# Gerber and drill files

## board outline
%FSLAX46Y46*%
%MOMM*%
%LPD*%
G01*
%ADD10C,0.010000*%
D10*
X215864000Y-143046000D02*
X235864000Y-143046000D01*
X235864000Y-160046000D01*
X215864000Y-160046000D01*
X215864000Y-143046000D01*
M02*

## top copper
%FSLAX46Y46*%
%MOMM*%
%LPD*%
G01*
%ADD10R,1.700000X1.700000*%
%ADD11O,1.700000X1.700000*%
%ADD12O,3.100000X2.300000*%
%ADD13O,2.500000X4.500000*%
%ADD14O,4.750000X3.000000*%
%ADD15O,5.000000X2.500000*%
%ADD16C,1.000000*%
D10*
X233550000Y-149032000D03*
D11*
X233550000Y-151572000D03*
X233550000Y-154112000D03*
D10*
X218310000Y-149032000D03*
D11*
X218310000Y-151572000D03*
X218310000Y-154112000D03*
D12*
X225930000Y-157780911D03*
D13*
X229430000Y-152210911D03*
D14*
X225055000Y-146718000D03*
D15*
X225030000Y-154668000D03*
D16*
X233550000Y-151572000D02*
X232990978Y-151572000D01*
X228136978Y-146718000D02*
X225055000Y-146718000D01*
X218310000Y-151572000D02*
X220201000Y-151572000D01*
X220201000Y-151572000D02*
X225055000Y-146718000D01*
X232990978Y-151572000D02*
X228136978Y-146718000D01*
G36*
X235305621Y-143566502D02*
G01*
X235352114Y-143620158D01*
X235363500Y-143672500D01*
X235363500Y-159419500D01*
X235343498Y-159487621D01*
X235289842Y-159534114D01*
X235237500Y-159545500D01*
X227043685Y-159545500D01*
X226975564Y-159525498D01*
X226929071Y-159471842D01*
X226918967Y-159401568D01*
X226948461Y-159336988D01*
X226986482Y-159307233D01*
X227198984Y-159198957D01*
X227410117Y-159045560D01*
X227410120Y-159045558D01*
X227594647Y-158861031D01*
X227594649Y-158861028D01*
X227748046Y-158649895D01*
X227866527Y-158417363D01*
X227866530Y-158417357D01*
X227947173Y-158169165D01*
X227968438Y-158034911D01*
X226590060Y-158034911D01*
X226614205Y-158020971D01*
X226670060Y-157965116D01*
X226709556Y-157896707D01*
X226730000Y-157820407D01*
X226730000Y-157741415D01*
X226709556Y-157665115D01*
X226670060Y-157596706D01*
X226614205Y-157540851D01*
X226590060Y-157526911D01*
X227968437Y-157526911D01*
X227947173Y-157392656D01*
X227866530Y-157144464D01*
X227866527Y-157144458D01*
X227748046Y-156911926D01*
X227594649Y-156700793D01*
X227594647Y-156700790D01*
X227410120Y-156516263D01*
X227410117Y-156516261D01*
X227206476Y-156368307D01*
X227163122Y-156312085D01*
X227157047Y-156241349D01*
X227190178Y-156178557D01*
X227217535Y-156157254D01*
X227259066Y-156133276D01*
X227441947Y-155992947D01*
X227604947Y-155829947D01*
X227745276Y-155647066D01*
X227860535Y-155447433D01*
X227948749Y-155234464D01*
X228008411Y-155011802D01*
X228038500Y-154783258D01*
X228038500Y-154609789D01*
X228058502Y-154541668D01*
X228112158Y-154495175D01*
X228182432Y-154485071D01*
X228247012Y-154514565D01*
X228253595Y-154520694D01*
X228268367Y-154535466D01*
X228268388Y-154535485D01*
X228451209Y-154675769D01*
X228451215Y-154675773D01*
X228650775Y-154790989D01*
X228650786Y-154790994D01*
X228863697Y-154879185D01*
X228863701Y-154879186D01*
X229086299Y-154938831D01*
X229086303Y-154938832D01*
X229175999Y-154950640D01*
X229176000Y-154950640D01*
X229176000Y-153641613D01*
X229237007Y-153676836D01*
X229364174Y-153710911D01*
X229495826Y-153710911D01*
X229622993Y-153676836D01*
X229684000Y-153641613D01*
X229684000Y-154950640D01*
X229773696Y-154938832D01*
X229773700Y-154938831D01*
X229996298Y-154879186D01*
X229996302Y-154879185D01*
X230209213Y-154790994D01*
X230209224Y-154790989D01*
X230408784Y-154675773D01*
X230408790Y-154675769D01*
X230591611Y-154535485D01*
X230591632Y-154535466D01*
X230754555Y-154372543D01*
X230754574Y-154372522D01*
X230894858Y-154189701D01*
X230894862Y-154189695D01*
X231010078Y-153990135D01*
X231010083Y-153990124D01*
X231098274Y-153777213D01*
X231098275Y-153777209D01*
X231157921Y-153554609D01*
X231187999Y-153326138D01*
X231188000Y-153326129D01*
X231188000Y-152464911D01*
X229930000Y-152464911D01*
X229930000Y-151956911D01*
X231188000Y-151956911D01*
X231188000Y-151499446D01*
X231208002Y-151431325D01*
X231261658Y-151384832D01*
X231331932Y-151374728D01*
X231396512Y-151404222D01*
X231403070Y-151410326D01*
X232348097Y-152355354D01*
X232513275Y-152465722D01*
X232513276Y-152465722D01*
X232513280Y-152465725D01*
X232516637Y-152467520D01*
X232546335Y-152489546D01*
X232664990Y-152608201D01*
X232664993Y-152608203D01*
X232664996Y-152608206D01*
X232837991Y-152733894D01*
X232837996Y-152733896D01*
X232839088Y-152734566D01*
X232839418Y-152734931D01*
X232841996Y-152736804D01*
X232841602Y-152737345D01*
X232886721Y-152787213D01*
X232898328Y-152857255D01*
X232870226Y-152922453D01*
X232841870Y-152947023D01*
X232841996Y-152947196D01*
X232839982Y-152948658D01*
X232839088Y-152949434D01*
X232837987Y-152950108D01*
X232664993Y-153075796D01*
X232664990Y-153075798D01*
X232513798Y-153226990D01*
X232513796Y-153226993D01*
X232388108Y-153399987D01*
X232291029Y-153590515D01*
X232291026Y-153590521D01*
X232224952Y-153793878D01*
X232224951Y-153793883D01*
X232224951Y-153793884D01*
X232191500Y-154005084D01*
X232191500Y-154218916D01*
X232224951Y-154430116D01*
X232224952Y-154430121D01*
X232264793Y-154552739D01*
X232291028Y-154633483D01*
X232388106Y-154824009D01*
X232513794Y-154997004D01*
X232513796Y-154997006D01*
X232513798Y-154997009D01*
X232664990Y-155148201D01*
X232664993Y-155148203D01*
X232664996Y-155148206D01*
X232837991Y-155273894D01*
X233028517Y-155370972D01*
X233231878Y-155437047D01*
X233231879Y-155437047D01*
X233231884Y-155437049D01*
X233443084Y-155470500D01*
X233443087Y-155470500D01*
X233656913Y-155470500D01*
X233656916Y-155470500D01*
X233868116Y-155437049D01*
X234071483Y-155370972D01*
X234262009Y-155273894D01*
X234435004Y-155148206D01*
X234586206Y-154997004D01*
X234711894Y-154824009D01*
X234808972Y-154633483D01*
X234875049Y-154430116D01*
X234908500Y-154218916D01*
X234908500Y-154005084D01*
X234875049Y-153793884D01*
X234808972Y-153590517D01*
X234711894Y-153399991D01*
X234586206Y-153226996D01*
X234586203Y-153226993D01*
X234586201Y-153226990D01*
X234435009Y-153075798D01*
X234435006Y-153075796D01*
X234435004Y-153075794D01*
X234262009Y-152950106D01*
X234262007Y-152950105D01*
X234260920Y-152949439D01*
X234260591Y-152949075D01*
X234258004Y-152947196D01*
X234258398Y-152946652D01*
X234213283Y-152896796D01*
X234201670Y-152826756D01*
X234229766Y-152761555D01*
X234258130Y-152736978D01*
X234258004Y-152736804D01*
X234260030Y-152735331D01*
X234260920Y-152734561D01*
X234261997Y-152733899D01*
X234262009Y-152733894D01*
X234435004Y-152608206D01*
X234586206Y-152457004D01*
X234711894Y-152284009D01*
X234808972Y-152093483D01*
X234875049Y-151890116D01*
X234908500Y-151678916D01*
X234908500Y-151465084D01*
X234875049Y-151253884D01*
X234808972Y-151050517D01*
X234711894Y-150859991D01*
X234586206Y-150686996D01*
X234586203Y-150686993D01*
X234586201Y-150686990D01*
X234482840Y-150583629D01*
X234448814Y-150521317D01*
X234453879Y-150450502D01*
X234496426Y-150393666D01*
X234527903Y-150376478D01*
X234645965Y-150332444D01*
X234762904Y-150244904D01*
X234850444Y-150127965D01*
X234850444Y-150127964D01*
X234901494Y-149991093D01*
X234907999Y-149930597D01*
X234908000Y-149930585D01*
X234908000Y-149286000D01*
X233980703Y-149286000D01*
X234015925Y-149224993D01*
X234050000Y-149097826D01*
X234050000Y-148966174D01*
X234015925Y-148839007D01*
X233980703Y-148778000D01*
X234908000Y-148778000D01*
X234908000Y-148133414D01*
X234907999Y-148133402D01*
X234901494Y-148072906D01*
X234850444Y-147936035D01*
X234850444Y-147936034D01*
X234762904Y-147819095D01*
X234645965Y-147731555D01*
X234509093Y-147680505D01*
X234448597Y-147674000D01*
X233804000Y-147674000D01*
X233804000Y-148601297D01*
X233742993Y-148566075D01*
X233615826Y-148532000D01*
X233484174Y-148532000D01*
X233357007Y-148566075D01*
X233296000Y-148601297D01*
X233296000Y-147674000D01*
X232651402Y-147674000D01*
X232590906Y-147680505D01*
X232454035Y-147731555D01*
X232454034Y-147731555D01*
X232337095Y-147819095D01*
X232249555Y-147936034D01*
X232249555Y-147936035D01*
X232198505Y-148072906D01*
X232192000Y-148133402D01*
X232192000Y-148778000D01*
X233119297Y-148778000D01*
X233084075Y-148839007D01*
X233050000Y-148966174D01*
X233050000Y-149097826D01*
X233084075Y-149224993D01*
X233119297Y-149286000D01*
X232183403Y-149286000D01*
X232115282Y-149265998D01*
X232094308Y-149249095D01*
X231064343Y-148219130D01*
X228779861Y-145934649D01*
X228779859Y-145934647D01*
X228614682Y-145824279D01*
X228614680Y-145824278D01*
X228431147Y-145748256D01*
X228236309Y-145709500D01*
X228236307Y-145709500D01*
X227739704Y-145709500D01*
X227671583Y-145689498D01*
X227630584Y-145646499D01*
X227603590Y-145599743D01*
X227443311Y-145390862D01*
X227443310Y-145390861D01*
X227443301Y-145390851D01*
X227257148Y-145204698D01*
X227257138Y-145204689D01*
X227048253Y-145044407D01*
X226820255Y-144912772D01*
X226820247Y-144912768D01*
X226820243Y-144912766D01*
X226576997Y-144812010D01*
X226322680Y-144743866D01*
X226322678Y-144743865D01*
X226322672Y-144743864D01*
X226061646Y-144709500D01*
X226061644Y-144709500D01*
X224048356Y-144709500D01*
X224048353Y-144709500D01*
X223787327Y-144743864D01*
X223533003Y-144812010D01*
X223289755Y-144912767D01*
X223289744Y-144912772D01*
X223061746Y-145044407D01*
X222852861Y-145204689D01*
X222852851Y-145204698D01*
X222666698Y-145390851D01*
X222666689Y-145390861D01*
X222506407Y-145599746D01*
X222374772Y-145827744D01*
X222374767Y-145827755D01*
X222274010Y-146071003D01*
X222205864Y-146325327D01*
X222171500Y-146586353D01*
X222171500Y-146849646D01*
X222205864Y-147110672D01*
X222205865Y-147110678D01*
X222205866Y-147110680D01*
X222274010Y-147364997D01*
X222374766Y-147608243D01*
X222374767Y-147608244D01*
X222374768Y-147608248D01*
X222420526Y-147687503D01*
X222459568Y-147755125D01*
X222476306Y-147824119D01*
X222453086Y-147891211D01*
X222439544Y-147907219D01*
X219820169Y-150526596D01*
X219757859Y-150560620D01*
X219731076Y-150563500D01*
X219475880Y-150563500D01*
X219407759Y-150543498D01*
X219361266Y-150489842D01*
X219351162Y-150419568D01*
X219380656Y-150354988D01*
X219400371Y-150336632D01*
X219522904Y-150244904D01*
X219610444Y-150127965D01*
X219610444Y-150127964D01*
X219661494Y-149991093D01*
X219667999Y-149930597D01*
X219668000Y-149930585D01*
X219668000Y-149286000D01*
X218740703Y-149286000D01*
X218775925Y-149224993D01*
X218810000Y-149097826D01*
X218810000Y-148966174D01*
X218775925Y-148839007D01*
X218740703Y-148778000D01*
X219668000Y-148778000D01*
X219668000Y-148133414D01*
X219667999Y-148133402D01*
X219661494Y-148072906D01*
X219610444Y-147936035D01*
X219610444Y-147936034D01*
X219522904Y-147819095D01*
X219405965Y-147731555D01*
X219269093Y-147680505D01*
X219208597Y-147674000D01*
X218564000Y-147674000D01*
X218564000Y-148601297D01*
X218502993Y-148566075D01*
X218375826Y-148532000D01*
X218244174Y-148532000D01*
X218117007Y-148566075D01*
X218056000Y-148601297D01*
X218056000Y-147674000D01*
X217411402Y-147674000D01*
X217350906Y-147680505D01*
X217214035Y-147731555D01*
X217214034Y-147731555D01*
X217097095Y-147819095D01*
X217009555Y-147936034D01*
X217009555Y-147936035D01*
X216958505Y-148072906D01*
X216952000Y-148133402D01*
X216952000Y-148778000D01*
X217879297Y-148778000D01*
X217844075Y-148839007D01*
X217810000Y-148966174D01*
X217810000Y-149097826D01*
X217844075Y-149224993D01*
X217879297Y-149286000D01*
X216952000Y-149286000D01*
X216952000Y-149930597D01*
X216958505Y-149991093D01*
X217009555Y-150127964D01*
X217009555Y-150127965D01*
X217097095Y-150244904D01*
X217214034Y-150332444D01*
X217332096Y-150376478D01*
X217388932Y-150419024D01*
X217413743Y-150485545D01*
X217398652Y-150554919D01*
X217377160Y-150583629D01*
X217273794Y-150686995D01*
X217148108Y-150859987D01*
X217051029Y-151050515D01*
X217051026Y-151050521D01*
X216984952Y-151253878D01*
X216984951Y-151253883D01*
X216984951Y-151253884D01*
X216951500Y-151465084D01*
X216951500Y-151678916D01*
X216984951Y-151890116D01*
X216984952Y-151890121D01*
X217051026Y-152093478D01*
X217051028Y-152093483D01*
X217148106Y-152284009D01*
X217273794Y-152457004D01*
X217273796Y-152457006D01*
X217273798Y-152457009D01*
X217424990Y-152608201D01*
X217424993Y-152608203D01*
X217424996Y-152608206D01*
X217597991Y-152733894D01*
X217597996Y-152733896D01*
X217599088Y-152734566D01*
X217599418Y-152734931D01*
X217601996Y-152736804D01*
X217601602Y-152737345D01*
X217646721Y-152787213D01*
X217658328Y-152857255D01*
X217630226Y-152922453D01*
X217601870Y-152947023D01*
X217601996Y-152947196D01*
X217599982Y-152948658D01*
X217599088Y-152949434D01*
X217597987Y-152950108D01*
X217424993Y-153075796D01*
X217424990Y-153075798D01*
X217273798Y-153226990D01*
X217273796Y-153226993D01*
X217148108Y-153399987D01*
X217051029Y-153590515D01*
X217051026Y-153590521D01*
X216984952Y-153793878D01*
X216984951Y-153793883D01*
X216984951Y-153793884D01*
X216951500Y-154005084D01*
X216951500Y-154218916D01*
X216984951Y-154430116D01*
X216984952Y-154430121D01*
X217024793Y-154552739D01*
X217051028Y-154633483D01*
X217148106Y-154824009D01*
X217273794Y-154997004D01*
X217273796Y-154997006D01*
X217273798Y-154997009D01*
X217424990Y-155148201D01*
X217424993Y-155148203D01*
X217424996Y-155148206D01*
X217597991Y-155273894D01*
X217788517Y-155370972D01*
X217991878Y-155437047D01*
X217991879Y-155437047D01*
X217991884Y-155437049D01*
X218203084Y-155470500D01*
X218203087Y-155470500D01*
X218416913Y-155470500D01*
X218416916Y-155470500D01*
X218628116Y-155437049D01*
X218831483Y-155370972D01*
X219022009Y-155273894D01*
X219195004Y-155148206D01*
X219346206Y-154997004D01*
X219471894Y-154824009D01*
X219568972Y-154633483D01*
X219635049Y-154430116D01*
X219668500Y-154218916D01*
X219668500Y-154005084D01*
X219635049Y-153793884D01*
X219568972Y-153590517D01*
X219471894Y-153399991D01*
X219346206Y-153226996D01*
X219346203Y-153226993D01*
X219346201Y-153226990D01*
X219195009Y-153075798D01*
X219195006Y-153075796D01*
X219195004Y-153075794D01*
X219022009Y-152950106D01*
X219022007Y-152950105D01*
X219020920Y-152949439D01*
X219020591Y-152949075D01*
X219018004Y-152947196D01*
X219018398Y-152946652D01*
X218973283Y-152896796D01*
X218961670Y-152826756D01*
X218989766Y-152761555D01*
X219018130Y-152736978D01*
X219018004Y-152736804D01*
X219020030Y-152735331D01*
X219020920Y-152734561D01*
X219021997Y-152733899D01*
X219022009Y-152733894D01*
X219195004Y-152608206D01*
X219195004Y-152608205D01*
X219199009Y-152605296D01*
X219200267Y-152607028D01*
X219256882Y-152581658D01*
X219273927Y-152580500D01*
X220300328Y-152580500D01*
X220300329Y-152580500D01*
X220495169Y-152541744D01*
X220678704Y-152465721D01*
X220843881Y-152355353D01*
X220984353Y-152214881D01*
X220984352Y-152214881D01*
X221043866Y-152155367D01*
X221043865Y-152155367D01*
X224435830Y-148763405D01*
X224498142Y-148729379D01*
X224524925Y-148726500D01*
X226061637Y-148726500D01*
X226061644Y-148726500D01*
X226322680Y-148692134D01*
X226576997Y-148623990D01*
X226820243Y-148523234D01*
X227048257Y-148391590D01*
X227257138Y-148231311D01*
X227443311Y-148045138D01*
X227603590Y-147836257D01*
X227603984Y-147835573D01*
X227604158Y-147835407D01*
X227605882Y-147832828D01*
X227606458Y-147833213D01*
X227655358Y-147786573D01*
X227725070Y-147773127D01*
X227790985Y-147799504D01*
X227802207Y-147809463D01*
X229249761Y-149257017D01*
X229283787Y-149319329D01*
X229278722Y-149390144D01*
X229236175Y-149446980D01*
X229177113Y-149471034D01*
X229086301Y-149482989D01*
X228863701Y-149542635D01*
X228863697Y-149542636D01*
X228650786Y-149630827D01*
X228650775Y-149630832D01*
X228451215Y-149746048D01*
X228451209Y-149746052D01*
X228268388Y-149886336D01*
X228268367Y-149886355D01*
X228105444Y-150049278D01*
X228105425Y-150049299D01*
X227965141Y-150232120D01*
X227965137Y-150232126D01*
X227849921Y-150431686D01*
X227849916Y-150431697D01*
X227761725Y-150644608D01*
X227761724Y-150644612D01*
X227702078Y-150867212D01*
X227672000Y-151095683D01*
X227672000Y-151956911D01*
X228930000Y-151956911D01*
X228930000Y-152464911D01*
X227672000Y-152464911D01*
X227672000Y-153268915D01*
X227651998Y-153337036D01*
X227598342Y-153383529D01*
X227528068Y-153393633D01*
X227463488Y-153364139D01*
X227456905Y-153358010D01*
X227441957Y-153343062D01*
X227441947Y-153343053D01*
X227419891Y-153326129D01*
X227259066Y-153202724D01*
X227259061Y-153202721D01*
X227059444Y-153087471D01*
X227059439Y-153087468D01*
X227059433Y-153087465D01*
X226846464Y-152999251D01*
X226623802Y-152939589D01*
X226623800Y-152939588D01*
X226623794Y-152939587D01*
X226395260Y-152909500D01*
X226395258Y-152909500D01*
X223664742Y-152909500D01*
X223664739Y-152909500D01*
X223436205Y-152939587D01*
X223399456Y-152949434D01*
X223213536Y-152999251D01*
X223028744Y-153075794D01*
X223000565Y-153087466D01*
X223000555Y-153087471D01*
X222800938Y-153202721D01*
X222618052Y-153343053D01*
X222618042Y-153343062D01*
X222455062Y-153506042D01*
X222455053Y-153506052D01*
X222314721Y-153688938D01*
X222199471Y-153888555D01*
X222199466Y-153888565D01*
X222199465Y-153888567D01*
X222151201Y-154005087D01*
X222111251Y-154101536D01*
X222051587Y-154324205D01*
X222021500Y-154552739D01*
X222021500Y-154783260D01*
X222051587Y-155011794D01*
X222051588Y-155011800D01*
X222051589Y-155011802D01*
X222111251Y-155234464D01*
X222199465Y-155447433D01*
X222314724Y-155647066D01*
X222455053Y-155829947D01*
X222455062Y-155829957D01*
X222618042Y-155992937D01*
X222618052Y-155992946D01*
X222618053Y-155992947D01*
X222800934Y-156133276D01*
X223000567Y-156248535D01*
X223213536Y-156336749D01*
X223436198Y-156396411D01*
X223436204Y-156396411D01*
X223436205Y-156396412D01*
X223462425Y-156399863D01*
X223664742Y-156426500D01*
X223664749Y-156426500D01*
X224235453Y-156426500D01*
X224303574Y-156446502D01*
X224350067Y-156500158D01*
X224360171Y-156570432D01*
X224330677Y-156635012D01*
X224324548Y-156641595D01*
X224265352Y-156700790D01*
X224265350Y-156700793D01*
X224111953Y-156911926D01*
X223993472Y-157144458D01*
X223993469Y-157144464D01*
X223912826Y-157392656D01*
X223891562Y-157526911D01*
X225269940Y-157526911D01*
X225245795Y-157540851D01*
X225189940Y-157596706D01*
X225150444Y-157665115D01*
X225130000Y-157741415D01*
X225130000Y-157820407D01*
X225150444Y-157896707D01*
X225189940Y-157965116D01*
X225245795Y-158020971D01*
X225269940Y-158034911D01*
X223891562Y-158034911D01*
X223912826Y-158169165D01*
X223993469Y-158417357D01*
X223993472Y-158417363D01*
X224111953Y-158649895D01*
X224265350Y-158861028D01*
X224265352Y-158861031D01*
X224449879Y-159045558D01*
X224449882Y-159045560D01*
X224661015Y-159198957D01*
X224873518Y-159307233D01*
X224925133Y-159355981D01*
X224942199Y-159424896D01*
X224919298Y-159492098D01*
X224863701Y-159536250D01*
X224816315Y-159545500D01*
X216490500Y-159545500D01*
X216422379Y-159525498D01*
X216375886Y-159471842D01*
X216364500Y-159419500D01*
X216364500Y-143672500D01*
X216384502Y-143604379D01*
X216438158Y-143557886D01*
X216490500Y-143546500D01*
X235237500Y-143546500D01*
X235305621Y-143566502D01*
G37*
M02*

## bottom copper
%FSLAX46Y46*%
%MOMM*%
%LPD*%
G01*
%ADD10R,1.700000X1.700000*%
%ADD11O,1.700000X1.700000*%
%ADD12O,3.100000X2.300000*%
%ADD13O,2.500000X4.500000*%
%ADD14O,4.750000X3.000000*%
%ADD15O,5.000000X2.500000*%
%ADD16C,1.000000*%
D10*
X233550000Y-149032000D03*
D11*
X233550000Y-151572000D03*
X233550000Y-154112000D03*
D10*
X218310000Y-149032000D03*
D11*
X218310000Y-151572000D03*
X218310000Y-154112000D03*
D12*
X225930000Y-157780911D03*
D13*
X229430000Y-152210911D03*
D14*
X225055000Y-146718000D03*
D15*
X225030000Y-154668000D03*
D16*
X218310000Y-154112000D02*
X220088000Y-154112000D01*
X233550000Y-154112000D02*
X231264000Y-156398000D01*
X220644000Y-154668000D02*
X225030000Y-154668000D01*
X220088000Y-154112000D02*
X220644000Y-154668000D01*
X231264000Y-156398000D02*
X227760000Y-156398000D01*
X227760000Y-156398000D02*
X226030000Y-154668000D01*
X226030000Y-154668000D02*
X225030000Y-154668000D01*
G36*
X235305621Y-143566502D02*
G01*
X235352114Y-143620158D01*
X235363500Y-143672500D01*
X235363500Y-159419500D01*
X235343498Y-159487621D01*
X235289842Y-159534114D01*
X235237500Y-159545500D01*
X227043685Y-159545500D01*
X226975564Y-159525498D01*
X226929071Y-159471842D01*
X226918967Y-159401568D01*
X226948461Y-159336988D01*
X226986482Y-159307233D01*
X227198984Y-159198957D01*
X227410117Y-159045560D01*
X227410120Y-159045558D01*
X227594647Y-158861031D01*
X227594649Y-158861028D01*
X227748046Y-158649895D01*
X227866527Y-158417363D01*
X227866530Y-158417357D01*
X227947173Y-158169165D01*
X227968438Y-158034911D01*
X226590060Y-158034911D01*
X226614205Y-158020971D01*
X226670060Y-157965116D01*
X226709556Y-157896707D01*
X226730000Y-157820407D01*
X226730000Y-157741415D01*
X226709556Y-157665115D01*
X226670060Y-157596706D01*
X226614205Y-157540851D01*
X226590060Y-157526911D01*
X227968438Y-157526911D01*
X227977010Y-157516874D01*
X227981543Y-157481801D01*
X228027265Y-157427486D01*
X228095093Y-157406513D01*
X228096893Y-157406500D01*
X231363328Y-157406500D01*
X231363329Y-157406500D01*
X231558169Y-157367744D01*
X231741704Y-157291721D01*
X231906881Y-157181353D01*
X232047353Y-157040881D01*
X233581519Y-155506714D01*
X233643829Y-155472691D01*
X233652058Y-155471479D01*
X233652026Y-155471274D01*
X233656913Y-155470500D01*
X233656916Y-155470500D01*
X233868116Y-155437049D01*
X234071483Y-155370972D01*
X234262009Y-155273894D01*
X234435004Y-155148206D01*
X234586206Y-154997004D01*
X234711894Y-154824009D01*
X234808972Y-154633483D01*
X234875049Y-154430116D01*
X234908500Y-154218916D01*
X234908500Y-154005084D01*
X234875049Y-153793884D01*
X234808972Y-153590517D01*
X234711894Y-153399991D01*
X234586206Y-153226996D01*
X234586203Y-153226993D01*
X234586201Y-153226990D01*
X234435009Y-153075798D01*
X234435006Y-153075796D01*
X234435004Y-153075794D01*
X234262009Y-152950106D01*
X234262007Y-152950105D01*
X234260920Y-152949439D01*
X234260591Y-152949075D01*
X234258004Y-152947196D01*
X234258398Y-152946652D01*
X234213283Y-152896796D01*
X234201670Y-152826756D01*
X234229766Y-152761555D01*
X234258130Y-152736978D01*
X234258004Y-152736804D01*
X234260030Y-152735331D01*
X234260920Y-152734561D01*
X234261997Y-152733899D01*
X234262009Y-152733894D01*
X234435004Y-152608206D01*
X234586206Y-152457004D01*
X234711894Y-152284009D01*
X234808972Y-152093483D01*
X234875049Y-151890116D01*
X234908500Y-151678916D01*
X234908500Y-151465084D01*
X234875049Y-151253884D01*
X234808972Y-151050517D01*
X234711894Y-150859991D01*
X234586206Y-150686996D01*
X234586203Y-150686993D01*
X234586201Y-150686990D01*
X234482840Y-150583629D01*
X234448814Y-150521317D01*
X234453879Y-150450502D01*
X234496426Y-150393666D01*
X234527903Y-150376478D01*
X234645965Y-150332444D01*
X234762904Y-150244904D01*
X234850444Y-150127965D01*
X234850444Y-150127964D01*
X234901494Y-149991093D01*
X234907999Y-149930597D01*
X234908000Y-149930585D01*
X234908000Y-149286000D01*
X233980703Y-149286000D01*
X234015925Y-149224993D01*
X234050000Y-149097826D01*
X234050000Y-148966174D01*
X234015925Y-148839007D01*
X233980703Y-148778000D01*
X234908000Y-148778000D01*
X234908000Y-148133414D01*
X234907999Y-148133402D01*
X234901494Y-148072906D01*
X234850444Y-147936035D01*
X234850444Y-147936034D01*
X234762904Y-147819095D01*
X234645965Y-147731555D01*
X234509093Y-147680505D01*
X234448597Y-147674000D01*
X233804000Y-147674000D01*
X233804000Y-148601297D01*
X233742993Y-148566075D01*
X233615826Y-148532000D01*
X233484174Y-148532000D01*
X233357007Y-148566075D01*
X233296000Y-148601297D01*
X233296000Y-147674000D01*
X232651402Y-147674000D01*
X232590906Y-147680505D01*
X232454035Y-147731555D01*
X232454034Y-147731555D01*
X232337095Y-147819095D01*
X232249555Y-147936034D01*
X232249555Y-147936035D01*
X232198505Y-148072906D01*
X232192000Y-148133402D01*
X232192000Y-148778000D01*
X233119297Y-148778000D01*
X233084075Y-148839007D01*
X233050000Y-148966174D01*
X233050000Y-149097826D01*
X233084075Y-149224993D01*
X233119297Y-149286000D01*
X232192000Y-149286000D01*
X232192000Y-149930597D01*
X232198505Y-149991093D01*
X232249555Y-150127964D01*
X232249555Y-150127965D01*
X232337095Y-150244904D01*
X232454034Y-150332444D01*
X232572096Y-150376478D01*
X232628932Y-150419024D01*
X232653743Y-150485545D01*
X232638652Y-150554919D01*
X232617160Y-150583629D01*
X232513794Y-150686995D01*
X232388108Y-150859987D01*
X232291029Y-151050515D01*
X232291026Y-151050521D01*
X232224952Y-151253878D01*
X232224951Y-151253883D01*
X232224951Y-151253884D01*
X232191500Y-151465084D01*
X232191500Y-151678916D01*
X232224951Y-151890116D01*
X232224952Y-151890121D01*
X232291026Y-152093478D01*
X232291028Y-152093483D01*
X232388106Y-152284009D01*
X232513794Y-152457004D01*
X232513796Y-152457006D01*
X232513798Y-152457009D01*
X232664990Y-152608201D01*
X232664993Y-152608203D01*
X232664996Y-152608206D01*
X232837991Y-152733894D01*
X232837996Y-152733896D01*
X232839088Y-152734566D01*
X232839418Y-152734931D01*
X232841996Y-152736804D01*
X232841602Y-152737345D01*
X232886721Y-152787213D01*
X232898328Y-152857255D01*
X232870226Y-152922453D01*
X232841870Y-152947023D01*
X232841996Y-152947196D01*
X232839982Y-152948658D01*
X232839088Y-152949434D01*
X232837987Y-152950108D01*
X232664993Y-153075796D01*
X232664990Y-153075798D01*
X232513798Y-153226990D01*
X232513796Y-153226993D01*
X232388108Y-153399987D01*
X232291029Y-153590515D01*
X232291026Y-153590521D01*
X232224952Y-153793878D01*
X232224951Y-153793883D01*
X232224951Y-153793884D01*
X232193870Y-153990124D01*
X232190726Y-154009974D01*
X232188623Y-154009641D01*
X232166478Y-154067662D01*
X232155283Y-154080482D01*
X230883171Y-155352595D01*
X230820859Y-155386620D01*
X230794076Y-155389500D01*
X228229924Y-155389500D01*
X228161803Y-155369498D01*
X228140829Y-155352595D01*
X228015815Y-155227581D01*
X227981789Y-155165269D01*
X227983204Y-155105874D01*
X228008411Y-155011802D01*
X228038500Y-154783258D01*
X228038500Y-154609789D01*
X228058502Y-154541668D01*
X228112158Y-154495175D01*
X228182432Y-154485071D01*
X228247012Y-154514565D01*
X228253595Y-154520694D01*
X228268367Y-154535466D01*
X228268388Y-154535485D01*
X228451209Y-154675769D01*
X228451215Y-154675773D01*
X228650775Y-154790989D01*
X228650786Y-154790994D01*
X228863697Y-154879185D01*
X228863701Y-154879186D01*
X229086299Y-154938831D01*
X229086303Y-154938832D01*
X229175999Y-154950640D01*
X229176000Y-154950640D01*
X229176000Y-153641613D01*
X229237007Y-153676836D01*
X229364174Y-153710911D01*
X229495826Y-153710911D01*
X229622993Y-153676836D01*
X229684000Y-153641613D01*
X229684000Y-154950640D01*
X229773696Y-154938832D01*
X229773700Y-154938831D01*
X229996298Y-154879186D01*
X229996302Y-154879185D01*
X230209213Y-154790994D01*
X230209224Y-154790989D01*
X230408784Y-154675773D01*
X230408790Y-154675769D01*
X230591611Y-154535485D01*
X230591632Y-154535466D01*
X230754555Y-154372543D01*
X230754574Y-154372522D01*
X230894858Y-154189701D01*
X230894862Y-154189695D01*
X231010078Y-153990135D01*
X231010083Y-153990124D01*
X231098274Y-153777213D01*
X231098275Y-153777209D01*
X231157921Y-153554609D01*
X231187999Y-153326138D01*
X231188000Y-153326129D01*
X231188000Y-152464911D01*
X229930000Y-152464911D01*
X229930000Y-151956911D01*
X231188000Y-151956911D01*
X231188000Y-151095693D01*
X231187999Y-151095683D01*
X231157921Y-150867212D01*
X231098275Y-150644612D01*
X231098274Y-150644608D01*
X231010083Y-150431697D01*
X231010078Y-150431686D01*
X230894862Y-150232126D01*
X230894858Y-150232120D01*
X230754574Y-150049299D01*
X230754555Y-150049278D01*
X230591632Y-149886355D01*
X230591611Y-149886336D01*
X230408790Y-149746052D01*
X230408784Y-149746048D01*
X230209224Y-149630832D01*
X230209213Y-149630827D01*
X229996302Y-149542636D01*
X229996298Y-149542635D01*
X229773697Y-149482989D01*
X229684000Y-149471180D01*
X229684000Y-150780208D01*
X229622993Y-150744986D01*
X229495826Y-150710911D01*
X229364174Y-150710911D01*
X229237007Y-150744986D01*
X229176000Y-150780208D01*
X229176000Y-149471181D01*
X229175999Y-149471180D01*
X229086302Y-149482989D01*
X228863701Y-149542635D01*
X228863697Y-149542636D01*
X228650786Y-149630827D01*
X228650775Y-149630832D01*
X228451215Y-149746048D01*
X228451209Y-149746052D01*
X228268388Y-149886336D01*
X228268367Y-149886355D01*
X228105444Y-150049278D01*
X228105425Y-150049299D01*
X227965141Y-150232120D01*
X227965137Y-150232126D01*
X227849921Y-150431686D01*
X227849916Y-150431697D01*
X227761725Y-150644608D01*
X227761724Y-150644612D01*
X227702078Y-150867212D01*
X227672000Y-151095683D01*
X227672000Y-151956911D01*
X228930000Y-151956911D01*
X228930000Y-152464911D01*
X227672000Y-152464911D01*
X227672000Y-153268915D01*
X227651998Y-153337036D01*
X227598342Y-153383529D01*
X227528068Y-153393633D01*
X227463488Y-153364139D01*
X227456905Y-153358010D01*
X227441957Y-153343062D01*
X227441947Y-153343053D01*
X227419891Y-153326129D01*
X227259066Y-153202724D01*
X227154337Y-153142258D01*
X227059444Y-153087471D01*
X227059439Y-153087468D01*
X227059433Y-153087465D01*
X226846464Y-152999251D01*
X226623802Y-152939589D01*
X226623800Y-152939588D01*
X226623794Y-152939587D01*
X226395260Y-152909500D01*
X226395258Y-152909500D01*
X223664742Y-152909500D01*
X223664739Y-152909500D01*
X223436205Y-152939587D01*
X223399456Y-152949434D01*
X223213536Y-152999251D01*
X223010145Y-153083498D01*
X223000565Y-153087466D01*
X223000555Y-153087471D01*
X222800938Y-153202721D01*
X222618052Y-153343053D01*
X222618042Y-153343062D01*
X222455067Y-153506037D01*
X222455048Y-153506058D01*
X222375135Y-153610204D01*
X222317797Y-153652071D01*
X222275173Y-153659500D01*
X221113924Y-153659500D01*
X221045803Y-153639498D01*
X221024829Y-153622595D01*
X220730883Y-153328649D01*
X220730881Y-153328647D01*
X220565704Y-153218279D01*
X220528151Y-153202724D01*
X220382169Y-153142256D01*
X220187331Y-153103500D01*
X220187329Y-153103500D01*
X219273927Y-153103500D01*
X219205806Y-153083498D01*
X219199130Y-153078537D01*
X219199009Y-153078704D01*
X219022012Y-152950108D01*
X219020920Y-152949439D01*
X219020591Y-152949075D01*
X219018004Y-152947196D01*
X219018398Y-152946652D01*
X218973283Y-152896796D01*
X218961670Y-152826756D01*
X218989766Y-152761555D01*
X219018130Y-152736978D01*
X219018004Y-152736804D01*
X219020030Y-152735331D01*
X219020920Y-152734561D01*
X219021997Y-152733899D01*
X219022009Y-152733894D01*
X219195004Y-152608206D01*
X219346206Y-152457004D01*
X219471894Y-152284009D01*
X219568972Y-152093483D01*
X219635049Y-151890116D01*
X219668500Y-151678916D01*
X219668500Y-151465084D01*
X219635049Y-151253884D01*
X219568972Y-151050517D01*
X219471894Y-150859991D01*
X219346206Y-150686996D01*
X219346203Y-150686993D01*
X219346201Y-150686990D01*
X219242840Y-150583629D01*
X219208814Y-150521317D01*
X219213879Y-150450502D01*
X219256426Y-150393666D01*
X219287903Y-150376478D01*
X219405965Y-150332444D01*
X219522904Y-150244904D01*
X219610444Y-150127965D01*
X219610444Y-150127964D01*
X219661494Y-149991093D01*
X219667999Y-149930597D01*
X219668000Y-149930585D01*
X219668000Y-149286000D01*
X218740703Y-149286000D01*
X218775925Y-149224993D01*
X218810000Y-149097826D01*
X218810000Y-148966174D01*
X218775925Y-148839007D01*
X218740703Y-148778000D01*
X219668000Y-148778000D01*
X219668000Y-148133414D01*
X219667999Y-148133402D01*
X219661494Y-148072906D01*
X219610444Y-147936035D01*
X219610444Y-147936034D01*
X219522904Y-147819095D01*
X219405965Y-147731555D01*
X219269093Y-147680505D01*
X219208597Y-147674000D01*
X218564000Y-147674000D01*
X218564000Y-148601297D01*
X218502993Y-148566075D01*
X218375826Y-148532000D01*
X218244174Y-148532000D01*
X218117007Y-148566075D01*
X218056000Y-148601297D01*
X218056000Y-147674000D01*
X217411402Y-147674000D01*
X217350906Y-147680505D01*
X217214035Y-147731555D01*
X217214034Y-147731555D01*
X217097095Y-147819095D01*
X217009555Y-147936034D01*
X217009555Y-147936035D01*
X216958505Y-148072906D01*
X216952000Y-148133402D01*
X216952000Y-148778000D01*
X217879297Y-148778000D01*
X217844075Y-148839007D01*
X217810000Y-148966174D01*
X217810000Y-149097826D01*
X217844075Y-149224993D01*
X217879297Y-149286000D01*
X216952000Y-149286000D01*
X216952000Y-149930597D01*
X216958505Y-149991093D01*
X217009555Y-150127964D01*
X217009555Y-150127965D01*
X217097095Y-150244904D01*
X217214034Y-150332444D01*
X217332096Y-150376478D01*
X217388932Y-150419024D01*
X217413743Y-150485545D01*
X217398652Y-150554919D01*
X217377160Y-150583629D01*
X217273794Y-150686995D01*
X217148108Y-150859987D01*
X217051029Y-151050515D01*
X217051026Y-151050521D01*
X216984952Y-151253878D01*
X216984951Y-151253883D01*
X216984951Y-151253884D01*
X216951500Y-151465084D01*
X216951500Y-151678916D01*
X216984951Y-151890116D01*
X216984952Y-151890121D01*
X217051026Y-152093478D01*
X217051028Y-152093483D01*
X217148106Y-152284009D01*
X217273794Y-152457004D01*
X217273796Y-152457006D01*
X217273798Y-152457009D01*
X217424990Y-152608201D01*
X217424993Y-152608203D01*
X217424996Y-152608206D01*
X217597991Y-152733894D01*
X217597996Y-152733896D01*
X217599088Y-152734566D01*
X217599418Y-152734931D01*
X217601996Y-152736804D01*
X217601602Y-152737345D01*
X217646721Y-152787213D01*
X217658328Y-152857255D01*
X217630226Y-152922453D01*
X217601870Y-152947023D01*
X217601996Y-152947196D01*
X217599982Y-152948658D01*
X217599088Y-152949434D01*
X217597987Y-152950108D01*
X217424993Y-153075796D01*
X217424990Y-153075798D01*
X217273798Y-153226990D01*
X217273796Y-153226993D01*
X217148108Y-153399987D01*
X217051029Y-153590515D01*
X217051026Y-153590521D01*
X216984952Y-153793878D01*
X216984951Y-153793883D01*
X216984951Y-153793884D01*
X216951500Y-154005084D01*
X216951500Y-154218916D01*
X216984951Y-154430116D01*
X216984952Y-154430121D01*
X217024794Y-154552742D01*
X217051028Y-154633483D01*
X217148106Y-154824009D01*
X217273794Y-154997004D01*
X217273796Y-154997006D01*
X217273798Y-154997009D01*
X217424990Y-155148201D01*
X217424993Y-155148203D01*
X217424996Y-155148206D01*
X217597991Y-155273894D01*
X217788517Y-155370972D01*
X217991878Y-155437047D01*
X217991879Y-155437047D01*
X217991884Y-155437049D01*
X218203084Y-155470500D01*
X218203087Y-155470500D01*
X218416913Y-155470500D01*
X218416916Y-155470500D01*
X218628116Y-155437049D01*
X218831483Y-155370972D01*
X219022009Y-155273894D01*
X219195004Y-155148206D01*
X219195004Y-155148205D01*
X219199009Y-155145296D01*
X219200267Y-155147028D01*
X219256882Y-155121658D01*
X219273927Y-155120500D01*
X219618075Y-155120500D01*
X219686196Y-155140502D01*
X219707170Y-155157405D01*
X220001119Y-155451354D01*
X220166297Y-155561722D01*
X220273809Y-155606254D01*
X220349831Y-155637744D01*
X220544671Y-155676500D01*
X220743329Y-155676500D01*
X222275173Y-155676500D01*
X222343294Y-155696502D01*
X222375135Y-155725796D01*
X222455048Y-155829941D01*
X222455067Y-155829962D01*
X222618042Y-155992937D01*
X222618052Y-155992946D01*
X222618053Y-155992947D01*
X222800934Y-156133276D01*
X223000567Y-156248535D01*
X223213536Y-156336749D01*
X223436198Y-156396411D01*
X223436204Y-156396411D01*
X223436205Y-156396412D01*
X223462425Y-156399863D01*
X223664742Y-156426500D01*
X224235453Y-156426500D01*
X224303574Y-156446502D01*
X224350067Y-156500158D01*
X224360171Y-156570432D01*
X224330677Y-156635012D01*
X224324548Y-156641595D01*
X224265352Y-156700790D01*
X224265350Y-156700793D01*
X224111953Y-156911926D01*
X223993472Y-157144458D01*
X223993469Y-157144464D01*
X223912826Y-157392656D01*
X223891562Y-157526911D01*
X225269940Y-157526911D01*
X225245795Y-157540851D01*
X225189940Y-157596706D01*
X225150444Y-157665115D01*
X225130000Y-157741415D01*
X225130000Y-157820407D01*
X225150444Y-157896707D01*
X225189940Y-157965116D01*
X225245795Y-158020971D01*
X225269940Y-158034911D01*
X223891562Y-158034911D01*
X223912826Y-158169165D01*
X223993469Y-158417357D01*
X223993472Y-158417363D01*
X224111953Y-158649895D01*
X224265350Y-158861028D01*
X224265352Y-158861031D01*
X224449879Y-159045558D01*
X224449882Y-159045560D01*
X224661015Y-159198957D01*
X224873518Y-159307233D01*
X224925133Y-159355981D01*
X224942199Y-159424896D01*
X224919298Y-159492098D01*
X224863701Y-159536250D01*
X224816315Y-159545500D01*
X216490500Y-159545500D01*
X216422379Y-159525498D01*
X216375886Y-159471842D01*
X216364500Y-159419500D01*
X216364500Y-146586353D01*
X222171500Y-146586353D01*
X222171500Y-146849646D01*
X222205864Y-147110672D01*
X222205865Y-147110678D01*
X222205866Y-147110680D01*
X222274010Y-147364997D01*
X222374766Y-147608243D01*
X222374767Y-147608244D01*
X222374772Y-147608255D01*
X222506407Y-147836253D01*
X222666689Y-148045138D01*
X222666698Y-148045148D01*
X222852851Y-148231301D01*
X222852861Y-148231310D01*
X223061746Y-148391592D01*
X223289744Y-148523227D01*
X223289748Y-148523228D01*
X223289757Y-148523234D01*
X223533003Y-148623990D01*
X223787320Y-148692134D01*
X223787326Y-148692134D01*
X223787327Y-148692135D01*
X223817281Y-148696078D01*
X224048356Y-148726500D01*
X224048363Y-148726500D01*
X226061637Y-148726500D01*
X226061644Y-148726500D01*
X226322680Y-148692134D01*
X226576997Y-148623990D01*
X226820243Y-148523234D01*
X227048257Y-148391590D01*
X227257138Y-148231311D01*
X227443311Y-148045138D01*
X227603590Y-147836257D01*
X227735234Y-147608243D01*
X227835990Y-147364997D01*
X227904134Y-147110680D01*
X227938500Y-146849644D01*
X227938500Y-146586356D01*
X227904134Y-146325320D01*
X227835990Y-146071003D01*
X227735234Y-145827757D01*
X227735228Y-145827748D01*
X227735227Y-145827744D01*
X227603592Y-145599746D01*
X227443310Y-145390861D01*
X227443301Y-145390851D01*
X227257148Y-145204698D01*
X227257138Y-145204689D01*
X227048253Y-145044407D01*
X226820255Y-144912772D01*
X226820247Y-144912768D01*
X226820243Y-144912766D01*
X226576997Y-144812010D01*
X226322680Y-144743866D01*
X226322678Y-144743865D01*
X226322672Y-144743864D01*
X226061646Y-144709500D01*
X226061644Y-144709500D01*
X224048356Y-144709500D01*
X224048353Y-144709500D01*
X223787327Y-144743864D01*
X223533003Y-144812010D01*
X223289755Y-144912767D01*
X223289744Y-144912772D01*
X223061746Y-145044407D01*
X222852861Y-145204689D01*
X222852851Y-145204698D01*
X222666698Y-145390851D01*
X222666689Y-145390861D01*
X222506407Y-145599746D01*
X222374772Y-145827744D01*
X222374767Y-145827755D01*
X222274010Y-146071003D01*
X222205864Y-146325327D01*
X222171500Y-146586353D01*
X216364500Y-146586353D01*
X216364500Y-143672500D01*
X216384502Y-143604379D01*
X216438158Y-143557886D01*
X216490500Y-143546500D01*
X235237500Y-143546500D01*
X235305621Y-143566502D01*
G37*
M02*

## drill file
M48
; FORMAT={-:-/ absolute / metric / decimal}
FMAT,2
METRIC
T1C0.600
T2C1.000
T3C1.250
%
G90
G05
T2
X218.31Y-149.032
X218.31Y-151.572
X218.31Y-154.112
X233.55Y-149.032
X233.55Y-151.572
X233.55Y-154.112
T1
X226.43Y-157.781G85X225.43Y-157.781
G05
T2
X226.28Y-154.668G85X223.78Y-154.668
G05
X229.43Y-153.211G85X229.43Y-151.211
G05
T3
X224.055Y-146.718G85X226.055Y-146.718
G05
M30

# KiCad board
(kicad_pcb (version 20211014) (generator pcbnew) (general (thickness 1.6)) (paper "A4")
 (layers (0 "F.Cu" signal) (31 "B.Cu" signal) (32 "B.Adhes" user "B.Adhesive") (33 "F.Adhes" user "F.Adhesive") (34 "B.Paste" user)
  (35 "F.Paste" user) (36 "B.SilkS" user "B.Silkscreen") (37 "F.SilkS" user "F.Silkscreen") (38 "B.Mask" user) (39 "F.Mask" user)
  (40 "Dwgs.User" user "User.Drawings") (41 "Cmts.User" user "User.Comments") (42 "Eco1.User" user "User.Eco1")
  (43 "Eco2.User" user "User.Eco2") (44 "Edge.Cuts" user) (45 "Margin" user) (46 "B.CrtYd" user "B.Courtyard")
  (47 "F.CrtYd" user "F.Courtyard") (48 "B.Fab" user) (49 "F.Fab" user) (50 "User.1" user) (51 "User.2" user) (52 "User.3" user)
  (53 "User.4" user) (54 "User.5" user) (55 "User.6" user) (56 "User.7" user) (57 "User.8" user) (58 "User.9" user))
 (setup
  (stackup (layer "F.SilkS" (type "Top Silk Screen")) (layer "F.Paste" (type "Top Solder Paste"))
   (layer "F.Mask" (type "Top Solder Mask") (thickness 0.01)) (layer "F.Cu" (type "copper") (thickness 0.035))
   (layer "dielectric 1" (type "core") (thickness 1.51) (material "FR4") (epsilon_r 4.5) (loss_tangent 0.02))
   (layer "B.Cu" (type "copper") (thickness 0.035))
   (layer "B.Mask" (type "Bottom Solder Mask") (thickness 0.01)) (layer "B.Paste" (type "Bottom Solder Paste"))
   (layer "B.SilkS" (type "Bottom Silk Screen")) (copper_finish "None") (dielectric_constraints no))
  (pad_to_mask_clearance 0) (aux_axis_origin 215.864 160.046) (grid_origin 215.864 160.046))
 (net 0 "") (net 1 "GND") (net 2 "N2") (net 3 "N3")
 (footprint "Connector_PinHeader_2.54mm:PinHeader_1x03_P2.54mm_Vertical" (layer "F.Cu") (at 233.55 149.032)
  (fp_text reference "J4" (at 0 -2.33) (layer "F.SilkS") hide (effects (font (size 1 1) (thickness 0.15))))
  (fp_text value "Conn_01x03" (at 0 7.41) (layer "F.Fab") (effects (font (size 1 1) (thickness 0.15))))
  (pad "1" thru_hole rect locked (at 0 0) (size 1.7 1.7) (drill 1) (layers *.Cu *.Mask) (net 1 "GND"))
  (pad "2" thru_hole oval locked (at 0 2.54) (size 1.7 1.7) (drill 1) (layers *.Cu *.Mask) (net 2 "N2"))
  (pad "3" thru_hole oval locked (at 0 5.08) (size 1.7 1.7) (drill 1) (layers *.Cu *.Mask) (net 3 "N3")))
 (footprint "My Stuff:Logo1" (layer "F.Cu") (at 224.382 150.805)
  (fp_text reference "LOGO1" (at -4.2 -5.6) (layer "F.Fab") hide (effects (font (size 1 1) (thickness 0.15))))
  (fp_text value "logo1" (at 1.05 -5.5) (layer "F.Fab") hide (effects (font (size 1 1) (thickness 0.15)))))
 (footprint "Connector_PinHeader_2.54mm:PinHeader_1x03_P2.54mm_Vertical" (layer "F.Cu") (at 218.31 149.032)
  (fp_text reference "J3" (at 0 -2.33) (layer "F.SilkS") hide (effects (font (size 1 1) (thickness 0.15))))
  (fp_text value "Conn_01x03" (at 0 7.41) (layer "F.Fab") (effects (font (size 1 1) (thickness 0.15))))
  (pad "1" thru_hole rect locked (at 0 0) (size 1.7 1.7) (drill 1) (layers *.Cu *.Mask) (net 1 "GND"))
  (pad "2" thru_hole oval locked (at 0 2.54) (size 1.7 1.7) (drill 1) (layers *.Cu *.Mask) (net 2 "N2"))
  (pad "3" thru_hole oval locked (at 0 5.08) (size 1.7 1.7) (drill 1) (layers *.Cu *.Mask) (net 3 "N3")))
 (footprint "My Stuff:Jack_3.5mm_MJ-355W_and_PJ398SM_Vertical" (layer "B.Cu") (at 225.93 151.318 180)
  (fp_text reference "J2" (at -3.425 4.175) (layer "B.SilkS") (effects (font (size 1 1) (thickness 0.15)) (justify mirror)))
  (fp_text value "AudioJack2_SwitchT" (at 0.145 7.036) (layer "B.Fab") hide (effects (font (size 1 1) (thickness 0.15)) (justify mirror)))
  (pad "S" thru_hole oval (at 0 -6.462911 180) (size 3.1 2.3) (drill oval 1.6 0.6) (layers *.Cu *.Mask) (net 1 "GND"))
  (pad "S" thru_hole oval (at -3.5 -0.892911 180) (size 2.5 4.5) (drill oval 1 3) (layers *.Cu *.Mask) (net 1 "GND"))
  (pad "T" thru_hole oval (at 0.875 4.6) (size 4.75 3) (drill oval 3.25 1.25) (layers *.Cu *.Mask) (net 2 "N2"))
  (pad "TN" thru_hole oval (at 0.9 -3.35 180) (size 5 2.5) (drill oval 3.5 1) (layers *.Cu *.Mask) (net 3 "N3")))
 (gr_rect (start 235.864 143.046) (end 215.864 160.046) (layer "Edge.Cuts") (width 0.01) (fill none))
 (segment (start 233.55 151.572) (end 232.990978 151.572) (width 1) (layer "F.Cu") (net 2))
 (segment (start 228.136978 146.718) (end 225.055 146.718) (width 1) (layer "F.Cu") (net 2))
 (segment (start 218.31 151.572) (end 220.201 151.572) (width 1) (layer "F.Cu") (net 2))
 (segment (start 220.201 151.572) (end 225.055 146.718) (width 1) (layer "F.Cu") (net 2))
 (segment (start 232.990978 151.572) (end 228.136978 146.718) (width 1) (layer "F.Cu") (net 2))
 (segment (start 218.31 154.112) (end 220.088 154.112) (width 1) (layer "B.Cu") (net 3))
 (segment (start 233.55 154.112) (end 231.264 156.398) (width 1) (layer "B.Cu") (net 3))
 (segment (start 220.644 154.668) (end 225.03 154.668) (width 1) (layer "B.Cu") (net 3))
 (segment (start 220.088 154.112) (end 220.644 154.668) (width 1) (layer "B.Cu") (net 3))
 (segment (start 231.264 156.398) (end 227.76 156.398) (width 1) (layer "B.Cu") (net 3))
 (segment (start 227.76 156.398) (end 226.03 154.668) (width 1) (layer "B.Cu") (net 3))
 (segment (start 226.03 154.668) (end 225.03 154.668) (width 1) (layer "B.Cu") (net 3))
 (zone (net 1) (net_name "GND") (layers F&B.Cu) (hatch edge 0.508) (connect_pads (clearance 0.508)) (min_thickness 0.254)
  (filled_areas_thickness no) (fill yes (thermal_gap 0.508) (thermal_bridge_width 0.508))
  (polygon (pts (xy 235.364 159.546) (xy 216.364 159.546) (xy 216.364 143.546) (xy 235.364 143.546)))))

